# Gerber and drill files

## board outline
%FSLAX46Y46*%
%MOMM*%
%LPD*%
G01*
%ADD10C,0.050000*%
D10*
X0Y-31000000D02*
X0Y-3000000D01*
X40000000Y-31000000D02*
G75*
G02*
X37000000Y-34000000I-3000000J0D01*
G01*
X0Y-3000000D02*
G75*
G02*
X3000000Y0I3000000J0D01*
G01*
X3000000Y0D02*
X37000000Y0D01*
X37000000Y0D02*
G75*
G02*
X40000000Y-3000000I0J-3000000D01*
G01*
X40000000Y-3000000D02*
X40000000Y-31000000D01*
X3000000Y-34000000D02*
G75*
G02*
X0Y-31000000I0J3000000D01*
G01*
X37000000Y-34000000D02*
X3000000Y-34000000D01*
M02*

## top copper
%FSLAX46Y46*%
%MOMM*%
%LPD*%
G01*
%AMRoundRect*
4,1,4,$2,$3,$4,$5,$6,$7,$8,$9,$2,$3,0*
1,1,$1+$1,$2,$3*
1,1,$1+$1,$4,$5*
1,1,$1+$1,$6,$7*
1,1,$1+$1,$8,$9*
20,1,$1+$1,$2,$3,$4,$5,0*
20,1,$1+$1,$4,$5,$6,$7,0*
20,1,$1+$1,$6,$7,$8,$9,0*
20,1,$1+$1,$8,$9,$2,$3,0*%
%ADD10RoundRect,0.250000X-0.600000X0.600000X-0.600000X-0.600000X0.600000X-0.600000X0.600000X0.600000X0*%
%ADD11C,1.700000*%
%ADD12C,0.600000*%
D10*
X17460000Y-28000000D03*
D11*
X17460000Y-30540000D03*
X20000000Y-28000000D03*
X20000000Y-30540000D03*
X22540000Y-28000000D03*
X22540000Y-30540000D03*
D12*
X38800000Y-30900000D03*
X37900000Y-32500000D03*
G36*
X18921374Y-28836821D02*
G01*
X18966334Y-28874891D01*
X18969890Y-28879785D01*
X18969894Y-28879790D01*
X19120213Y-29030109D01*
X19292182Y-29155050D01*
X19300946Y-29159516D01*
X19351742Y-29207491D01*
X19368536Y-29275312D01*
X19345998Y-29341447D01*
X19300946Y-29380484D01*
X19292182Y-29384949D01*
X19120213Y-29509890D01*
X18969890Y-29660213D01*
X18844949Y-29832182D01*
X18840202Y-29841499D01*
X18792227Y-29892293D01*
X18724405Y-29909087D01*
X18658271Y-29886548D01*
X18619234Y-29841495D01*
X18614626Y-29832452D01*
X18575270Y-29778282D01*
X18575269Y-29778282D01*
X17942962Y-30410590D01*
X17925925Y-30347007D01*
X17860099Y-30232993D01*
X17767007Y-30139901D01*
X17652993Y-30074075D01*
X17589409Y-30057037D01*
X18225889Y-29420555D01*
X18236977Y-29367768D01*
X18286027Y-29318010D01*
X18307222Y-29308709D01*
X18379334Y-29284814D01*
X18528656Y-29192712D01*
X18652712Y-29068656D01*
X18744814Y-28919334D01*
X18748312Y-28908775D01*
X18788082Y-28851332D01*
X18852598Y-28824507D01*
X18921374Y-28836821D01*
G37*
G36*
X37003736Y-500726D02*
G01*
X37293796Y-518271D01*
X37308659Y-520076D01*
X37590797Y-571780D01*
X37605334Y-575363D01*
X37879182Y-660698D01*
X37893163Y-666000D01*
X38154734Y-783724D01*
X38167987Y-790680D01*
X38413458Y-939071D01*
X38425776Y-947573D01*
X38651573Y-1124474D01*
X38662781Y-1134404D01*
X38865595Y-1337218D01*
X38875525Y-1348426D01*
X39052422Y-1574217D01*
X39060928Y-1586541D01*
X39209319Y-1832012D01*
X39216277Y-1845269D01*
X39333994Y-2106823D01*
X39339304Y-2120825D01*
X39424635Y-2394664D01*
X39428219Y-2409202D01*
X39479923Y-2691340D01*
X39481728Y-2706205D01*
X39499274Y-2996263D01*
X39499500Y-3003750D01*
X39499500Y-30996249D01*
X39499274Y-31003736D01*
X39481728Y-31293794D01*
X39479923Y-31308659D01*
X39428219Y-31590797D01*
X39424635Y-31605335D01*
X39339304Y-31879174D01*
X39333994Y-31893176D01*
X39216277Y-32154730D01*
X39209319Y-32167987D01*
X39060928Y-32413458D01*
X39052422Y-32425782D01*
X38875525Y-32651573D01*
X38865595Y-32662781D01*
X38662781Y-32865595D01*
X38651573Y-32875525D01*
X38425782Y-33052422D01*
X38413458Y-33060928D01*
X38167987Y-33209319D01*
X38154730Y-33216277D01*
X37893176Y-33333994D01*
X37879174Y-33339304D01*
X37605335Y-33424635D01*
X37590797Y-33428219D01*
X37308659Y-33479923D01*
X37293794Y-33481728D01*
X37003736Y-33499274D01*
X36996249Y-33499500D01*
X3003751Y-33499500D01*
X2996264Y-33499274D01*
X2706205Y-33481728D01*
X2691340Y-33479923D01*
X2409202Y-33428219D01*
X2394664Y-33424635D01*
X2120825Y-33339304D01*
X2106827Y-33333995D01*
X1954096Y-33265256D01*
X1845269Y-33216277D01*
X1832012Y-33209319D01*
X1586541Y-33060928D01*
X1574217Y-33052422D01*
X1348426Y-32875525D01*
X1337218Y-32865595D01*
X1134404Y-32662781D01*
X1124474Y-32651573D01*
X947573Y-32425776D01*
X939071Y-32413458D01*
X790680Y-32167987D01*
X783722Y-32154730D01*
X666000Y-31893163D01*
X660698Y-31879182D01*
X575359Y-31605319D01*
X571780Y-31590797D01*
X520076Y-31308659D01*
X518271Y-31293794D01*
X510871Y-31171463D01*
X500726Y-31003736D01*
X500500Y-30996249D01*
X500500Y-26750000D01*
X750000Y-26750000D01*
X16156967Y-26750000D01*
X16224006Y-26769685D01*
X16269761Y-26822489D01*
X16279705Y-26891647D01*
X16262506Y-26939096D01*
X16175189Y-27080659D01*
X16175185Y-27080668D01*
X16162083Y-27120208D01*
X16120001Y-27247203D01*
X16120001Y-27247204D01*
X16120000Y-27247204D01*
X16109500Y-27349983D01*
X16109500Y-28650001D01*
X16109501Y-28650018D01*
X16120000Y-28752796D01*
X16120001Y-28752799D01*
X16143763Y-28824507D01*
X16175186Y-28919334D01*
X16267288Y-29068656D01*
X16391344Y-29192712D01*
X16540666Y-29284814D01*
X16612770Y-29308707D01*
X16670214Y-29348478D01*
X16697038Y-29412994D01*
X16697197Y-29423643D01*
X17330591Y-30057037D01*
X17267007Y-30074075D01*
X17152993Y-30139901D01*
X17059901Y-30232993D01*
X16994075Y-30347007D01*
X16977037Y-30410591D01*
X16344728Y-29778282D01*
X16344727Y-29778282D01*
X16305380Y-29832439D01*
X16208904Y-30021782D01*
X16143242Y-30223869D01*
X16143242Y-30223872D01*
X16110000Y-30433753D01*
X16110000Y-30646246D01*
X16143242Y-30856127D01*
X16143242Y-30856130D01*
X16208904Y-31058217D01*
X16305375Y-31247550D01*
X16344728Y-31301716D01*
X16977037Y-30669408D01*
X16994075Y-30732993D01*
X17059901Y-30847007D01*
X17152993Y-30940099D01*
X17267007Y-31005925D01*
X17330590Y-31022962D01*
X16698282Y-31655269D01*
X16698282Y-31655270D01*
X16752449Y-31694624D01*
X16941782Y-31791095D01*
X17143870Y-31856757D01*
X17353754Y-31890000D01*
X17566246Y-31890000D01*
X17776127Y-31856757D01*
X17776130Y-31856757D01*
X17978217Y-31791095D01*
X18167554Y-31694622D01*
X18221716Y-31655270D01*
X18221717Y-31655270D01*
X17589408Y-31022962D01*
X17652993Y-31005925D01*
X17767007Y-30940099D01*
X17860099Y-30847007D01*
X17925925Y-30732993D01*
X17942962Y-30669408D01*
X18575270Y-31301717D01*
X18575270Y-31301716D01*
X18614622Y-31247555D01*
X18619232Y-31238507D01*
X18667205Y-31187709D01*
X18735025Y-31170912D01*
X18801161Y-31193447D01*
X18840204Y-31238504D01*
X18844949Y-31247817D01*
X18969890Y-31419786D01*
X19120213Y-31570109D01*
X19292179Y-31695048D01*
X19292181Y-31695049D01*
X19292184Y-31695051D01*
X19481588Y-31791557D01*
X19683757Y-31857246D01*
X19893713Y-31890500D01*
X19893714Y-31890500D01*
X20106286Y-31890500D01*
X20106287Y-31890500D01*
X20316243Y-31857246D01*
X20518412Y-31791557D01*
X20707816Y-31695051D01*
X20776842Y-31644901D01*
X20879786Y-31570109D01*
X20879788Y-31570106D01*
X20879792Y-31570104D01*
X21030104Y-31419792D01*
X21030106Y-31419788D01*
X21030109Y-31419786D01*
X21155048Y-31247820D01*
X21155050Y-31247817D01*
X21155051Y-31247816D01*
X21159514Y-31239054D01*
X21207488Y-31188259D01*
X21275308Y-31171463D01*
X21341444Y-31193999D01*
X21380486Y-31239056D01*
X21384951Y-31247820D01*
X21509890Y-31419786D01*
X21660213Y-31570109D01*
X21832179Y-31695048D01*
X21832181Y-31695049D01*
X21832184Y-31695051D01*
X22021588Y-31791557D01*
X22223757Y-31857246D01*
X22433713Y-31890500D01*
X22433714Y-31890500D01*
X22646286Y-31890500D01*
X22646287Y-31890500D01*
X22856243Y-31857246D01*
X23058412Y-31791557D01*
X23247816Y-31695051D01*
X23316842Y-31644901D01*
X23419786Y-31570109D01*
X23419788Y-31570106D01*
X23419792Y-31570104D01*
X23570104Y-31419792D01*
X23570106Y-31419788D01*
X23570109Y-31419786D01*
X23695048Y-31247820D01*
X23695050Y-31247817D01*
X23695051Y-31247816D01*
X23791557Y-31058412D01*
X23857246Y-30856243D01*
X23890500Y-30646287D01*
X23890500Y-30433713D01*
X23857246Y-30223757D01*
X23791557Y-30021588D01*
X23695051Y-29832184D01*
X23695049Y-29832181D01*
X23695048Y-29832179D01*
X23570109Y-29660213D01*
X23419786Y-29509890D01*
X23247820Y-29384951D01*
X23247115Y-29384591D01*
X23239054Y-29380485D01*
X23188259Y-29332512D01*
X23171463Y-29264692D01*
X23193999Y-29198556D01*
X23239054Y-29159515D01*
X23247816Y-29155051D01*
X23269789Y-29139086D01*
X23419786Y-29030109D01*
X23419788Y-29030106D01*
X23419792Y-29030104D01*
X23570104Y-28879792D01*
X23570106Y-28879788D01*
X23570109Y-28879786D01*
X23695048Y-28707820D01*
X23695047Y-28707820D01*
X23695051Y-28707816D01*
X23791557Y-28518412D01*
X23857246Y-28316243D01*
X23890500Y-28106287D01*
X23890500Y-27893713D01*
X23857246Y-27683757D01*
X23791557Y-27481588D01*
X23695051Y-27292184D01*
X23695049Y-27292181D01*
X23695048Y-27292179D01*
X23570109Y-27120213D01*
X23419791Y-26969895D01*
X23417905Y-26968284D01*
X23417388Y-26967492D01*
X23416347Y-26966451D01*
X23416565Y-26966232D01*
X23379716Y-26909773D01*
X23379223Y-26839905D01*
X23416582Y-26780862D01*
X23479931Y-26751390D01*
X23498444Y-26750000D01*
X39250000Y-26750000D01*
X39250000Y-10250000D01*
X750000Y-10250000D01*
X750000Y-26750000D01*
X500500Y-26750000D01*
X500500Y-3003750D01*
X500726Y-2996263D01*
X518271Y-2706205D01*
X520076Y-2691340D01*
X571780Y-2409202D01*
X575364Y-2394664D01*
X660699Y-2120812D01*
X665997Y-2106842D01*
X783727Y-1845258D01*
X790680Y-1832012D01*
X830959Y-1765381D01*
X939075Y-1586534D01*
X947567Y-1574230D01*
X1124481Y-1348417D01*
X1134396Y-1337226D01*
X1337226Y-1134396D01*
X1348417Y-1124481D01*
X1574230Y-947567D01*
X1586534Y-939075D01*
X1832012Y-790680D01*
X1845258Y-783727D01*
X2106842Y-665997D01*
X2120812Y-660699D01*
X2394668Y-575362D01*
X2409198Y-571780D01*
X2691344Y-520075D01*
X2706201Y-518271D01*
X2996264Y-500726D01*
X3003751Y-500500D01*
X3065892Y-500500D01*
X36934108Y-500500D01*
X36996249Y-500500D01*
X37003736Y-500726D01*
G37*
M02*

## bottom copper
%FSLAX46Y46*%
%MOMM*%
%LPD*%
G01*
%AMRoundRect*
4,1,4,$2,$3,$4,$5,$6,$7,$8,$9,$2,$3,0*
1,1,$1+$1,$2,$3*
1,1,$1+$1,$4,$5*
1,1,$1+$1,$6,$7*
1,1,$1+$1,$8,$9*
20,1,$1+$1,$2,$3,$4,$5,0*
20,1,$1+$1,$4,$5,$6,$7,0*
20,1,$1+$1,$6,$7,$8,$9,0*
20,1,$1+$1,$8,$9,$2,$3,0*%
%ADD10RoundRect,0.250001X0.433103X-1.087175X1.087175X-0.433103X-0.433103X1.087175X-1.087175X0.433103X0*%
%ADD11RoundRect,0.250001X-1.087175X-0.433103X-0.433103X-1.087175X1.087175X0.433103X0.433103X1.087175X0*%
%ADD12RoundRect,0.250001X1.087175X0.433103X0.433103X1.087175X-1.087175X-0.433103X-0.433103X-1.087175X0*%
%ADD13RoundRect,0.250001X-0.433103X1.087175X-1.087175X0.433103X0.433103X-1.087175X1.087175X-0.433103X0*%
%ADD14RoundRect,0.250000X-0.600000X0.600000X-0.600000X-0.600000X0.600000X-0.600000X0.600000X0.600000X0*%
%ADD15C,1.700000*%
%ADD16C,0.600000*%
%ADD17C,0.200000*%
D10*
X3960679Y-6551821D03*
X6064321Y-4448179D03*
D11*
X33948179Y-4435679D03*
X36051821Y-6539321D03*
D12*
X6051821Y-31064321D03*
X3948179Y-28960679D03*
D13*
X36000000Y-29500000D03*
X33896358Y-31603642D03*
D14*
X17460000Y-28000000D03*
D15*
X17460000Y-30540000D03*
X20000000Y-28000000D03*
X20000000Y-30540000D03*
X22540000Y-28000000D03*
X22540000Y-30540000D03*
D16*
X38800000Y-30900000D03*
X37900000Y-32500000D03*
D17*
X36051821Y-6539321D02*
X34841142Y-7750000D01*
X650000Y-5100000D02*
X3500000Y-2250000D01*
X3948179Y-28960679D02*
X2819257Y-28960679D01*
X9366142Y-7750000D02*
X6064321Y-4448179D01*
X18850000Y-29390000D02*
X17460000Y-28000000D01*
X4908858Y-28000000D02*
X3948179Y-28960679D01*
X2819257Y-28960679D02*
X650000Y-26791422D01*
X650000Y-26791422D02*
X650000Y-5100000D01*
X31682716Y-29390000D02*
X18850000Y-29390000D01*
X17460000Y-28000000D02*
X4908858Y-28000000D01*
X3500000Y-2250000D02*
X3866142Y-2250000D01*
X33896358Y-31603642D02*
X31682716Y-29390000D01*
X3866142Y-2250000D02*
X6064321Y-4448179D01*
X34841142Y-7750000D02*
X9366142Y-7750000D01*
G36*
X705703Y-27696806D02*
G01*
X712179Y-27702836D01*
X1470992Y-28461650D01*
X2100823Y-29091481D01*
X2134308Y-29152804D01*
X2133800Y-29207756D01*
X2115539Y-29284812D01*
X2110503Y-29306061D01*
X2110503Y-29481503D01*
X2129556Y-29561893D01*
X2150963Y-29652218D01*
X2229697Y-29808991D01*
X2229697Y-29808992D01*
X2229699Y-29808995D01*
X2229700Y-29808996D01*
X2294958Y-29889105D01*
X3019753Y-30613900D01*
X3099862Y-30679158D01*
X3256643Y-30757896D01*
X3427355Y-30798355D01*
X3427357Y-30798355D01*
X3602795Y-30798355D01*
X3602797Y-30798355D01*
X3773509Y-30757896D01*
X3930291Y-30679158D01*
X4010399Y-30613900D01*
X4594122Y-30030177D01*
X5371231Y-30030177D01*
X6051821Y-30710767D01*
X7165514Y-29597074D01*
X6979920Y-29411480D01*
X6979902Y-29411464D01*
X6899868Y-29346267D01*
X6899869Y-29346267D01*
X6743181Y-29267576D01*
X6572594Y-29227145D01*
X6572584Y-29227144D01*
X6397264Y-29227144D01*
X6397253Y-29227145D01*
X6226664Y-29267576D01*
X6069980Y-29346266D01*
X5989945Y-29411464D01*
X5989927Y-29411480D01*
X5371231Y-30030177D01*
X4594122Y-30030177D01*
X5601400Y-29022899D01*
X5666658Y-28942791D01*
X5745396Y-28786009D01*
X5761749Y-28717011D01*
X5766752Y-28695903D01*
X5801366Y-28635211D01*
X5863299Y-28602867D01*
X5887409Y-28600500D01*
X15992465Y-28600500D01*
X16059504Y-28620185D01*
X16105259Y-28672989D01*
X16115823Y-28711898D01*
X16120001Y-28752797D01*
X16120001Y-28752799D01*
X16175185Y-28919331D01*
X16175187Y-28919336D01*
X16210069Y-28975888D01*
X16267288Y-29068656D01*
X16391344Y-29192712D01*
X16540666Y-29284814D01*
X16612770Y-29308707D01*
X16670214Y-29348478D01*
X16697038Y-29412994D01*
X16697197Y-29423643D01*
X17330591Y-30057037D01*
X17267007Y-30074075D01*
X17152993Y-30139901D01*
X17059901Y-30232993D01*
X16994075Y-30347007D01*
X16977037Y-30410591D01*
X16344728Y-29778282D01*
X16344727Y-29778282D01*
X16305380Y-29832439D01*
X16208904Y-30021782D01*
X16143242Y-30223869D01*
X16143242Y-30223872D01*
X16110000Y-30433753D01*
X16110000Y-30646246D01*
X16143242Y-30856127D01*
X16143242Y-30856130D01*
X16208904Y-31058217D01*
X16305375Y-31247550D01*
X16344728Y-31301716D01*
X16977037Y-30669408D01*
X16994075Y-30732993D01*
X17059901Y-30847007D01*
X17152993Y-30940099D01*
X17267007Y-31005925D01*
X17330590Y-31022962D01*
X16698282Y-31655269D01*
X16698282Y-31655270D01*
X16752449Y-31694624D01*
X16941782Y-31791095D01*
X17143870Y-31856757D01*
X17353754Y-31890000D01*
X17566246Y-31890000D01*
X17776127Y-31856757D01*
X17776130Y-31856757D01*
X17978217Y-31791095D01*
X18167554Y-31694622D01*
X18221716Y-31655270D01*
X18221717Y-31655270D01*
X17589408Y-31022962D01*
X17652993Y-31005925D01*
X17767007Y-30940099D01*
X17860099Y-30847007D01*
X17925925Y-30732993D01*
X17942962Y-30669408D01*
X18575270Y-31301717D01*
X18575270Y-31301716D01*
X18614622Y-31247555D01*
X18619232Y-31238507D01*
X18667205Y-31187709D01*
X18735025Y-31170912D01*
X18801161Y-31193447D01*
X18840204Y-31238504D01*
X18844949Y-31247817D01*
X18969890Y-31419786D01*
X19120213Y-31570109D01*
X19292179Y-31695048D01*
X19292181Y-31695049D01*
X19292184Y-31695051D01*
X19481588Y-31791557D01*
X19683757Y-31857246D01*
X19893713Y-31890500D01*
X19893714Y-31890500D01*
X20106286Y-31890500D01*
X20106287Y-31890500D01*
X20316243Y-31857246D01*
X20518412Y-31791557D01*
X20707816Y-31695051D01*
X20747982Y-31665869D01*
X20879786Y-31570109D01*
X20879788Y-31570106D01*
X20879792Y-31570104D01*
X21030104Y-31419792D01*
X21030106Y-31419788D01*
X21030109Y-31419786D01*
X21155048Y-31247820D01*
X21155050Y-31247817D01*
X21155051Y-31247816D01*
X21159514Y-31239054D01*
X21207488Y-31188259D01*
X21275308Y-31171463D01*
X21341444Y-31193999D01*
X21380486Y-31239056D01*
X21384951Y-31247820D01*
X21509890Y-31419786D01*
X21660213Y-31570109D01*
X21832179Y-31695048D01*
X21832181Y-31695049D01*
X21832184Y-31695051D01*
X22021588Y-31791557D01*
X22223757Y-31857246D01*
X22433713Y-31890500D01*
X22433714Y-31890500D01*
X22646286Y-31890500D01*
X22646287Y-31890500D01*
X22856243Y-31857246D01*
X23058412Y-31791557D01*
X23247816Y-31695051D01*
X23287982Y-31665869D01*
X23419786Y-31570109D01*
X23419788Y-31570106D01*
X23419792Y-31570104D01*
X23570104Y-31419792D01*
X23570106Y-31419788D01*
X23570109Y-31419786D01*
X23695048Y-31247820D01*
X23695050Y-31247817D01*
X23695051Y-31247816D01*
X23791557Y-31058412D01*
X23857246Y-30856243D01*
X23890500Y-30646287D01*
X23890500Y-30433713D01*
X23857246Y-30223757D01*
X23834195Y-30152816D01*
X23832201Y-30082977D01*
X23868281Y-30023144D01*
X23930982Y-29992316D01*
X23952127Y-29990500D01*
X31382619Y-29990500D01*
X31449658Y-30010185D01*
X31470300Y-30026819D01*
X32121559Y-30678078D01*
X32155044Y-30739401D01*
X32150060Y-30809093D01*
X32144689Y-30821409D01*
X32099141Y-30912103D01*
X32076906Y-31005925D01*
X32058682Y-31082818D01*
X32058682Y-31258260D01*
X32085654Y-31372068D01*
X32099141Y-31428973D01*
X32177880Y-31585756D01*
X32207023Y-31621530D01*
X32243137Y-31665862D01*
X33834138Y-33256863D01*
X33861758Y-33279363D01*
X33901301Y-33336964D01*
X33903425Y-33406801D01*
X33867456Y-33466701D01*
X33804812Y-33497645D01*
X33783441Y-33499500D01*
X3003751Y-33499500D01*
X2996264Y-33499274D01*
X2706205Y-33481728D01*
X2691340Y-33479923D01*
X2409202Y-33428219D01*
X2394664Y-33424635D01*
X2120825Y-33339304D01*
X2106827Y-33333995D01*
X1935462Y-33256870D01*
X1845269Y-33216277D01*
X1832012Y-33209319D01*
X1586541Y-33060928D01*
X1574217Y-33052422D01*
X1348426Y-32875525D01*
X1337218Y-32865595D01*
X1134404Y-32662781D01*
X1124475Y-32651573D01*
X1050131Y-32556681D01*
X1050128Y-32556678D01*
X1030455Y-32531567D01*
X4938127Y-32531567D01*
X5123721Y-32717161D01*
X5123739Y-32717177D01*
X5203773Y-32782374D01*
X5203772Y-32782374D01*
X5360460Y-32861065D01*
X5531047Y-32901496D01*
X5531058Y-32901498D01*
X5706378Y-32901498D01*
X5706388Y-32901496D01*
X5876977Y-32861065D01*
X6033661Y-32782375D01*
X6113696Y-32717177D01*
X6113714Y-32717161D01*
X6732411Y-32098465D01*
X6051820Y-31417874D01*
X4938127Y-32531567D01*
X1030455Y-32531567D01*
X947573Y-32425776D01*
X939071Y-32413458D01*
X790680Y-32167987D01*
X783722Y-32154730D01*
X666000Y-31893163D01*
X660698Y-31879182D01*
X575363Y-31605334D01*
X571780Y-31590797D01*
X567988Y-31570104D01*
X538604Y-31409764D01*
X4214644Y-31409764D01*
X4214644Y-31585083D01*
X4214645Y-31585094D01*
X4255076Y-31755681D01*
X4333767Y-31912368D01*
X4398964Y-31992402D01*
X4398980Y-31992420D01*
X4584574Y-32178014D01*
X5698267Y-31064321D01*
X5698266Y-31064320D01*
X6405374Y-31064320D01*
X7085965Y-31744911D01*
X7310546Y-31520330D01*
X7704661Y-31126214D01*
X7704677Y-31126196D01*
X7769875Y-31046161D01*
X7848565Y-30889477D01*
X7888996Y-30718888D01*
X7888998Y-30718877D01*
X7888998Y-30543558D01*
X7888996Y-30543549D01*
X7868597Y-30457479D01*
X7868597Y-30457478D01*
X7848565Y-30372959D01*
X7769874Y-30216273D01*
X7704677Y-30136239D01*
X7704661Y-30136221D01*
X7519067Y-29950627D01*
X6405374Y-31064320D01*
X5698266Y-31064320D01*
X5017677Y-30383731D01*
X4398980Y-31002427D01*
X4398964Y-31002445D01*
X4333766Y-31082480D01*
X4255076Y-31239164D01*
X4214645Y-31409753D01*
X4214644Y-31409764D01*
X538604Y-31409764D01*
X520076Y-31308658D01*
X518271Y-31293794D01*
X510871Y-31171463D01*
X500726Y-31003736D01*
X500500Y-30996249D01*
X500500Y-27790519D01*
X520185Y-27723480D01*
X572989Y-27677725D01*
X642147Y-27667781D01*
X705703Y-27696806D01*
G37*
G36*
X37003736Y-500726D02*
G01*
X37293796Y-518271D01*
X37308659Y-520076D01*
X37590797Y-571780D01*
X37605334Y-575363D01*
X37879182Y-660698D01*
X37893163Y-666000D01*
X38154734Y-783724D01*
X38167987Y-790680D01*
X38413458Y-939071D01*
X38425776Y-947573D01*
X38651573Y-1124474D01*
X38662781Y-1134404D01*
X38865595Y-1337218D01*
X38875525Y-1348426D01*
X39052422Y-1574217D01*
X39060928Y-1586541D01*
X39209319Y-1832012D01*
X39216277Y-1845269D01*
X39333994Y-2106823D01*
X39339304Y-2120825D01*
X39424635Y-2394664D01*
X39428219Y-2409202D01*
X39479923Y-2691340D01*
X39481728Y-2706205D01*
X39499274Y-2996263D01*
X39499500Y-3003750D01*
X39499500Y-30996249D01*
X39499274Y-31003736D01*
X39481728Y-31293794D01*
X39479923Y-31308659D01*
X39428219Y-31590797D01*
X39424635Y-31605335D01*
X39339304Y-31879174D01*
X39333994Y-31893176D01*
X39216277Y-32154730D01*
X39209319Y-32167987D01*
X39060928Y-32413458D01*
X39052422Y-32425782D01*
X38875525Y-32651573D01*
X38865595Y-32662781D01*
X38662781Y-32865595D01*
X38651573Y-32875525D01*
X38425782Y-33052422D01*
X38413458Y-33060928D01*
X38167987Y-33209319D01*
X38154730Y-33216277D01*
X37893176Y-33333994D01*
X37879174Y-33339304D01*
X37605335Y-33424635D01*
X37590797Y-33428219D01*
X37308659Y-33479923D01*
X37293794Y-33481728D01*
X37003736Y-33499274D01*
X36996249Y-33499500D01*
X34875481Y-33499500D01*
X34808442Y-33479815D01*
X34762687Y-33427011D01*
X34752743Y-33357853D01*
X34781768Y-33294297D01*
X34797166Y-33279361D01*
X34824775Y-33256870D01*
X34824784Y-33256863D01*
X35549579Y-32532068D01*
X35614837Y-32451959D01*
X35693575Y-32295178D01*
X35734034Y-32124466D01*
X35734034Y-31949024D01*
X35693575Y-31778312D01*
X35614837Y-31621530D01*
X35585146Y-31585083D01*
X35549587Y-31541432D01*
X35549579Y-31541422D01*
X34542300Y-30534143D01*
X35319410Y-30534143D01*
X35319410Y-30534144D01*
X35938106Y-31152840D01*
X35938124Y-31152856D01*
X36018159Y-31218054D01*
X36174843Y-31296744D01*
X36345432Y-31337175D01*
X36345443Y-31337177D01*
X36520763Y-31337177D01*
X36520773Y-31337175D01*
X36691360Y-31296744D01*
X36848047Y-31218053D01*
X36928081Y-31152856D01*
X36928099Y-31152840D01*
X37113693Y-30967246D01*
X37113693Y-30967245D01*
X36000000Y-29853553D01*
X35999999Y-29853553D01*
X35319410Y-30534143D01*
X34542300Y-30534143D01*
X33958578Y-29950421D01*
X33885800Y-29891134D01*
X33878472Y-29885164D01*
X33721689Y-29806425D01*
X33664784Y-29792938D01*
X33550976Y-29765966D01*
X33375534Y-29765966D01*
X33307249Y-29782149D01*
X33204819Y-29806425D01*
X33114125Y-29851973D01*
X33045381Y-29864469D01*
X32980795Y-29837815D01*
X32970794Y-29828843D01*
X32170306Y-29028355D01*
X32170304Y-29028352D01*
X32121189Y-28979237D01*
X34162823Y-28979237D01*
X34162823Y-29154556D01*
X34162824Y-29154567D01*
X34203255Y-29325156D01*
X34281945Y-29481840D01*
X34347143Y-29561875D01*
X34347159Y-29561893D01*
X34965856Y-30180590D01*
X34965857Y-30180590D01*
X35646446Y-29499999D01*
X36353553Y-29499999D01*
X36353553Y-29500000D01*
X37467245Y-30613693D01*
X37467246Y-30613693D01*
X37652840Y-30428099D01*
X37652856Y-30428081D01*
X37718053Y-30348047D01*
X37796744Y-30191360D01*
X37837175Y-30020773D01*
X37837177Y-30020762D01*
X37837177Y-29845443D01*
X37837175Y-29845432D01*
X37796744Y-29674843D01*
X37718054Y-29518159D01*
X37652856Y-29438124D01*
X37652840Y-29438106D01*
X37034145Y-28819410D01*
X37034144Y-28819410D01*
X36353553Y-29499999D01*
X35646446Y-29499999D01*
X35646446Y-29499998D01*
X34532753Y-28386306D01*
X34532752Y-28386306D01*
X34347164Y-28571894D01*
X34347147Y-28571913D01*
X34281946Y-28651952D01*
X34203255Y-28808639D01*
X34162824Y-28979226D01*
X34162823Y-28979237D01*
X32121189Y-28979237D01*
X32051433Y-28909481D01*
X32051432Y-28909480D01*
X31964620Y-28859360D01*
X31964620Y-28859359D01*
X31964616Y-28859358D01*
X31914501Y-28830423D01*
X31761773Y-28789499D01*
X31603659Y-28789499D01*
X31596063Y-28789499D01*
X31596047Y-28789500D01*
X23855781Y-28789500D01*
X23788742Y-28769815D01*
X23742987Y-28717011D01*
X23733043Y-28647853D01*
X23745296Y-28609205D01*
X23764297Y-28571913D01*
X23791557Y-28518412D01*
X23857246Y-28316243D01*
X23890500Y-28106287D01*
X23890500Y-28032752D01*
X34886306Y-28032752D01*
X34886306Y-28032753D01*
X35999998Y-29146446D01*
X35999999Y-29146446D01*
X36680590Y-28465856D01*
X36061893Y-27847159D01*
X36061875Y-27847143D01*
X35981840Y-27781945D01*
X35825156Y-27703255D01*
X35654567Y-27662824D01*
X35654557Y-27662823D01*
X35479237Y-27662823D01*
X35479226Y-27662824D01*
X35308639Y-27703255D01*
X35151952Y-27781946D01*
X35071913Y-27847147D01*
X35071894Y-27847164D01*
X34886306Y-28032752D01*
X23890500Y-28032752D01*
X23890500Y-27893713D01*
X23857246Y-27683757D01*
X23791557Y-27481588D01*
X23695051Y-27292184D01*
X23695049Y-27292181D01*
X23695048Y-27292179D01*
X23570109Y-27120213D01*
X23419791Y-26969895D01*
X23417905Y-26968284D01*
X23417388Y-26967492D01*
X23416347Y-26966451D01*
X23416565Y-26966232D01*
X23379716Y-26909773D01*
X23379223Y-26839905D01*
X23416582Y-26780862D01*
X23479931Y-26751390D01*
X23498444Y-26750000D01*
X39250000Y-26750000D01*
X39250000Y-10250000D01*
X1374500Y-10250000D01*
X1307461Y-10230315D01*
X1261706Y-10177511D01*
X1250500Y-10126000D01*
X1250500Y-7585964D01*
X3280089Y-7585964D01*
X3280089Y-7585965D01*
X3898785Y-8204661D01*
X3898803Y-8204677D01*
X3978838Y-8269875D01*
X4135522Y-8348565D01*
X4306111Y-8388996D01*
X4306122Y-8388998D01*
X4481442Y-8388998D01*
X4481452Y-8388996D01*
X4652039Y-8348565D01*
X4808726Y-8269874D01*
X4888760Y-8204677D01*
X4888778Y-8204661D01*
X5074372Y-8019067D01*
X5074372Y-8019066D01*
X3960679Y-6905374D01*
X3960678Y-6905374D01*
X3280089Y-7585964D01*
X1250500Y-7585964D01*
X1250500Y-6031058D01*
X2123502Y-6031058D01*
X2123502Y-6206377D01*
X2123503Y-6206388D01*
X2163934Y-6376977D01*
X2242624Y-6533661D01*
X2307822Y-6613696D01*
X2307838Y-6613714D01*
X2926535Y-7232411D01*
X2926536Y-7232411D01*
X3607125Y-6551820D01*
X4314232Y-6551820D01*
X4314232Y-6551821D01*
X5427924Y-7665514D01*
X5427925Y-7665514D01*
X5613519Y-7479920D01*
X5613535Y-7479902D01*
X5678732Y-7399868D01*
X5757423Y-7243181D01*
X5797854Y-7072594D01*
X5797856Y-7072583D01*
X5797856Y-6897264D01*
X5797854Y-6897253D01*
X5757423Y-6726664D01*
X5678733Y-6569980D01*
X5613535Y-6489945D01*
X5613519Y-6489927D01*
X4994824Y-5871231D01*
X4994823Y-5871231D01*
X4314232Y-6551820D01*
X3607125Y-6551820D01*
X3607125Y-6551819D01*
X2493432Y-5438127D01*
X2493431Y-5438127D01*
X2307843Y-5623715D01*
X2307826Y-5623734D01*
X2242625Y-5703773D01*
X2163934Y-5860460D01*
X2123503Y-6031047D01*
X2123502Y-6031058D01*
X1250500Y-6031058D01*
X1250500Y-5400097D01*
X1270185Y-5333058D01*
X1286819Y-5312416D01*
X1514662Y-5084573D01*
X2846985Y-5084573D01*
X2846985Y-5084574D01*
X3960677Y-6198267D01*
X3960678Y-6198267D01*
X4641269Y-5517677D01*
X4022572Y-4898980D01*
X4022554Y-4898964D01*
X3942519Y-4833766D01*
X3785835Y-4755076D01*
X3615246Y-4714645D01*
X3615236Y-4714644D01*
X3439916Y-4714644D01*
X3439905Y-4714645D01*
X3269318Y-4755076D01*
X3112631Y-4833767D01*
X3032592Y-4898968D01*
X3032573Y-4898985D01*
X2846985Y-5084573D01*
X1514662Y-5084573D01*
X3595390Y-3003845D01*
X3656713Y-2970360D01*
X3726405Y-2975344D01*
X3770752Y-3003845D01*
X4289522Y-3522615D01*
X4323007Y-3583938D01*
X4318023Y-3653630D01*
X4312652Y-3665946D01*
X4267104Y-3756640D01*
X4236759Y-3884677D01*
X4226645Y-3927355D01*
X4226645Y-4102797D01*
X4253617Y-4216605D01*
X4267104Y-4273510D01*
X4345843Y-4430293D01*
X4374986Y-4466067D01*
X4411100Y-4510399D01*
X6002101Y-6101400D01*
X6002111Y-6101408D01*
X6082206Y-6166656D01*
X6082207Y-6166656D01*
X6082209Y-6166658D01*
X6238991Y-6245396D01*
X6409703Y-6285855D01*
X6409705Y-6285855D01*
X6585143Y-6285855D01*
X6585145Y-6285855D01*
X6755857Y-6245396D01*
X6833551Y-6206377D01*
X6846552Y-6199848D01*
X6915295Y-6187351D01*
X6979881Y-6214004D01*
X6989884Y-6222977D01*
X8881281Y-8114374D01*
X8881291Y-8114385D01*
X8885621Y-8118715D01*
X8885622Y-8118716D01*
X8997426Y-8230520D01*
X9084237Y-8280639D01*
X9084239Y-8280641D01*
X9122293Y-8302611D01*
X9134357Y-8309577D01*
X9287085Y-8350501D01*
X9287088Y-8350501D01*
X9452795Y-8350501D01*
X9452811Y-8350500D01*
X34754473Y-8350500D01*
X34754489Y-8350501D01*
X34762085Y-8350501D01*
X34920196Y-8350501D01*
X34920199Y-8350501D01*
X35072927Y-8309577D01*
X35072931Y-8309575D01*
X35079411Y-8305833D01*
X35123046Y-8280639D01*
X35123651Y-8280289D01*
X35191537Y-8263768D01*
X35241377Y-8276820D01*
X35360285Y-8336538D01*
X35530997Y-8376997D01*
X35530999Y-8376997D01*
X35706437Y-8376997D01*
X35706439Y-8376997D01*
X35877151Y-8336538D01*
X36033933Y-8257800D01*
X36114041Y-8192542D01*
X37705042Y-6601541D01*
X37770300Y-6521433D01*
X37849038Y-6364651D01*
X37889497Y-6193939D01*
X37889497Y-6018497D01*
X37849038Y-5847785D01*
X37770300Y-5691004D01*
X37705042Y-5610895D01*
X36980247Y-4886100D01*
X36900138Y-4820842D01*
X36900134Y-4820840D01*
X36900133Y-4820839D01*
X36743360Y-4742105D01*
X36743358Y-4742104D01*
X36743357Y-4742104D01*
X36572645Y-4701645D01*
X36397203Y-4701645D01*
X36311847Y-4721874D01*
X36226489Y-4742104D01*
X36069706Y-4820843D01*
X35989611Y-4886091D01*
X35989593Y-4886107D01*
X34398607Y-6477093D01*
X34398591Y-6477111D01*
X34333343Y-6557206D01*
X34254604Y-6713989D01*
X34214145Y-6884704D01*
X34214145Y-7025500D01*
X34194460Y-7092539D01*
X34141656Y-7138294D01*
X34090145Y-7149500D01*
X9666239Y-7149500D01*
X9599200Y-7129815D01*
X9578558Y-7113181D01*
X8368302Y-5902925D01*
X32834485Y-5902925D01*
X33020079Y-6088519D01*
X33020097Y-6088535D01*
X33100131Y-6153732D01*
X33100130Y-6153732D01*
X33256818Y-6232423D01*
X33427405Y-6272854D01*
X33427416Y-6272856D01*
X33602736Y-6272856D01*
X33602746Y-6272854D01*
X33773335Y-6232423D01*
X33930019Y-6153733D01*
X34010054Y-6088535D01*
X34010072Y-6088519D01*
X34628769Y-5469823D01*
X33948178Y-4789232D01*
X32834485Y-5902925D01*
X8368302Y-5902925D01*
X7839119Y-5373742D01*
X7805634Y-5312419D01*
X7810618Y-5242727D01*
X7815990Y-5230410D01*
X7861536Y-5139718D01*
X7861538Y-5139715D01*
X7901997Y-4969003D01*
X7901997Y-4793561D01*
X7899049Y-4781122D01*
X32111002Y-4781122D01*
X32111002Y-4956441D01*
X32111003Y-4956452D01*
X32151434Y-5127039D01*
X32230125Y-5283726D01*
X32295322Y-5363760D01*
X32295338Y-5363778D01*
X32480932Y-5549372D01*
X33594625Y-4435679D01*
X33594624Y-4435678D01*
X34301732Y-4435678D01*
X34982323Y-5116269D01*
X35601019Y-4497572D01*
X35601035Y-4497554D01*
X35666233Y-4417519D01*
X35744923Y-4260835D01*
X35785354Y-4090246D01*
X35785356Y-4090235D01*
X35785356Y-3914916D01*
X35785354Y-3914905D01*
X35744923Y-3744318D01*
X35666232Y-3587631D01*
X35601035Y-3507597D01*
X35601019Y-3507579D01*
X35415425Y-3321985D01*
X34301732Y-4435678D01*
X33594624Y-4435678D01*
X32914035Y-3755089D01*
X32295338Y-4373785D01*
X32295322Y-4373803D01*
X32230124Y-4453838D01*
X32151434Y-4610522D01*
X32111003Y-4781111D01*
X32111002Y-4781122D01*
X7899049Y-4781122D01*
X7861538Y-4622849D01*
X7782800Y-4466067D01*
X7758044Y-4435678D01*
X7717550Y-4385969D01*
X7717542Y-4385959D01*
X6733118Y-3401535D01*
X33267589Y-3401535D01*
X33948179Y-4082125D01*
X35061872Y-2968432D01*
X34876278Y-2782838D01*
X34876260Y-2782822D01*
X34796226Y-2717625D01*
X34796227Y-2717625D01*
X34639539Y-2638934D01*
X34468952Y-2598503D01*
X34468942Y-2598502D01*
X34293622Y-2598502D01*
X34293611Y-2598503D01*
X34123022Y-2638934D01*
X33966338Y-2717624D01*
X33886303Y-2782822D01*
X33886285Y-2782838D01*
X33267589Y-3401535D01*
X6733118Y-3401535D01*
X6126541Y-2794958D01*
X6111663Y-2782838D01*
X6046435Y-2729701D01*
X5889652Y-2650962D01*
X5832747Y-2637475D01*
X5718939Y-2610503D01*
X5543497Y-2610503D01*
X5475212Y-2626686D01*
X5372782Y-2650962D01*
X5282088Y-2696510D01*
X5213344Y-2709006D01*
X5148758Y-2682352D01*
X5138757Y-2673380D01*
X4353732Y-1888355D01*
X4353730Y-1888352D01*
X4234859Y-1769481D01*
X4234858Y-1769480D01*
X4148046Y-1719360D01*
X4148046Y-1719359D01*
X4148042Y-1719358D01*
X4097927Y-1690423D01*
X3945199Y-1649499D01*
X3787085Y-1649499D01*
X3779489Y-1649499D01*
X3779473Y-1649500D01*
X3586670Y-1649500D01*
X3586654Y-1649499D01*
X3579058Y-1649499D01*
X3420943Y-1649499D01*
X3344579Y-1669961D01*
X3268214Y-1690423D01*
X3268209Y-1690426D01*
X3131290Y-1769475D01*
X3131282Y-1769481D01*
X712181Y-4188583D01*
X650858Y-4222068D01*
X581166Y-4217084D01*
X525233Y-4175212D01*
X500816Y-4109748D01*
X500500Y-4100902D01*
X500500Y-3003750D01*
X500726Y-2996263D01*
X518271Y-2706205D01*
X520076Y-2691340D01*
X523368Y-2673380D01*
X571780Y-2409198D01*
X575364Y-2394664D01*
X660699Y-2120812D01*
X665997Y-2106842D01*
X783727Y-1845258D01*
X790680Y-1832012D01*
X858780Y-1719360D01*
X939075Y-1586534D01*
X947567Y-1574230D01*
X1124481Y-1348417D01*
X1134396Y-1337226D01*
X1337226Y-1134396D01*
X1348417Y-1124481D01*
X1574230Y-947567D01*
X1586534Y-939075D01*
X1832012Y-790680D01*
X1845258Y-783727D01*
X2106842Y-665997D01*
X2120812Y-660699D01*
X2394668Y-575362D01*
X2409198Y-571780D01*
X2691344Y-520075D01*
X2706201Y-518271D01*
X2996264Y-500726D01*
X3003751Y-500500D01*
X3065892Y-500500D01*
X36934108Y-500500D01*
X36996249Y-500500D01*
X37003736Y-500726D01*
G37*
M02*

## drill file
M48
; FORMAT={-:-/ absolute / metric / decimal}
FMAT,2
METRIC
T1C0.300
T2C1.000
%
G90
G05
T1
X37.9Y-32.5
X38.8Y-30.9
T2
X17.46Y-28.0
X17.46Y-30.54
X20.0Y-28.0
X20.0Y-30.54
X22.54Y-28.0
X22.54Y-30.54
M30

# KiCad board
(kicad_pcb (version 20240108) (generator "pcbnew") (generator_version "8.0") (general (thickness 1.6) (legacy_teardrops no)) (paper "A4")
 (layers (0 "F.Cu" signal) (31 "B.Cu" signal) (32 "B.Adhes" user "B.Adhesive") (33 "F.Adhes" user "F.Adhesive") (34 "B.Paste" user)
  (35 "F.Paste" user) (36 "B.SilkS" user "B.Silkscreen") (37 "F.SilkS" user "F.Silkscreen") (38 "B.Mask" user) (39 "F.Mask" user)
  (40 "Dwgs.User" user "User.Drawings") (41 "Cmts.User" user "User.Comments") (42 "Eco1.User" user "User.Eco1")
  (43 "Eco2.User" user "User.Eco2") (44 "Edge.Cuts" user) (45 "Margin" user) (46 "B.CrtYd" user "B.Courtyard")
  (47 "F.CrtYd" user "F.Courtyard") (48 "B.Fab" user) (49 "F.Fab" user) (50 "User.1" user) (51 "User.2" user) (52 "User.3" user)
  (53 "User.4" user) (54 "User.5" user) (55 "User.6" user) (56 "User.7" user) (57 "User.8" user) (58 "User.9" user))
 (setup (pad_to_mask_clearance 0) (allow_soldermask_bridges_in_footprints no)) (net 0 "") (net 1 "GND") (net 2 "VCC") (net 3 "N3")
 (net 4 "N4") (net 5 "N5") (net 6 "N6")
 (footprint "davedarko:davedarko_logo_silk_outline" (layer "F.Cu") (at 36.5 30)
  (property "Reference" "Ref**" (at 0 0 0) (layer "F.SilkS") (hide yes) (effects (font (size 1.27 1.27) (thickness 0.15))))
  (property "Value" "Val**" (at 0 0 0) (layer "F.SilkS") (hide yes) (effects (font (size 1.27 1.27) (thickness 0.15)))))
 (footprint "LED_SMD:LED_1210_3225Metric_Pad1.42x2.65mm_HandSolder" (layer "B.Cu") (at 5.0125 5.5 45)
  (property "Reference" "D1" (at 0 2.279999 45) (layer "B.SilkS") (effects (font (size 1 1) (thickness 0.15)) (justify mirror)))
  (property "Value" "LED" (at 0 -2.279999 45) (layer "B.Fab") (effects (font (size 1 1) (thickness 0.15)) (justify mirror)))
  (pad "1" smd roundrect (at -1.4875 0 45) (size 1.425 2.65) (layers "B.Cu" "B.Paste" "B.Mask") (roundrect_rratio 0.175439) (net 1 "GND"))
  (pad "2" smd roundrect (at 1.4875 0 45) (size 1.425 2.65) (layers "B.Cu" "B.Paste" "B.Mask") (roundrect_rratio 0.175439) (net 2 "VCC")))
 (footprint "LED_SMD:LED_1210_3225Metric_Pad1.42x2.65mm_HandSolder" (layer "B.Cu") (at 35 5.4875 -45)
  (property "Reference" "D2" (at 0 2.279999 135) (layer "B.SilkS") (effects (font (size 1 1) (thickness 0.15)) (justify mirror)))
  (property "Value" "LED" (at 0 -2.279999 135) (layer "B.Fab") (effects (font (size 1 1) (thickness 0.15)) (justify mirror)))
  (pad "1" smd roundrect (at -1.4875 0 315) (size 1.425 2.65) (layers "B.Cu" "B.Paste" "B.Mask") (roundrect_rratio 0.175439) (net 1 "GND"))
  (pad "2" smd roundrect (at 1.4875 0 315) (size 1.425 2.65) (layers "B.Cu" "B.Paste" "B.Mask") (roundrect_rratio 0.175439) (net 2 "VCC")))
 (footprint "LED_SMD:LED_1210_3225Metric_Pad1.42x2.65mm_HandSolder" (layer "B.Cu") (at 5 30.0125 135)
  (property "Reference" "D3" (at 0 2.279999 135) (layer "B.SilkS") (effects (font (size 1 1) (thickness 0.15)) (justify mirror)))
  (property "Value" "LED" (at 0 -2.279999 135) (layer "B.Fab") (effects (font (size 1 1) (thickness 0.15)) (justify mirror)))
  (pad "1" smd roundrect (at -1.4875 0 135) (size 1.425 2.65) (layers "B.Cu" "B.Paste" "B.Mask") (roundrect_rratio 0.175439) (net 1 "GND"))
  (pad "2" smd roundrect (at 1.4875 0 135) (size 1.425 2.65) (layers "B.Cu" "B.Paste" "B.Mask") (roundrect_rratio 0.175439) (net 2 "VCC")))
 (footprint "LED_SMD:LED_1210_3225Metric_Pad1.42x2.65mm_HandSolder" (layer "B.Cu") (at 34.948179 30.551821 -135)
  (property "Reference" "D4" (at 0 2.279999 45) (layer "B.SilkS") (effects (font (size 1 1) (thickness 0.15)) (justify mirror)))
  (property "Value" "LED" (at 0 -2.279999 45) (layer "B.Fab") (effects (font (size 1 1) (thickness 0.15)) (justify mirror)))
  (pad "1" smd roundrect (at -1.4875 0 225) (size 1.425 2.65) (layers "B.Cu" "B.Paste" "B.Mask") (roundrect_rratio 0.175439) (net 1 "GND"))
  (pad "2" smd roundrect (at 1.4875 0 225) (size 1.425 2.65) (layers "B.Cu" "B.Paste" "B.Mask") (roundrect_rratio 0.175439) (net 2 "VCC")))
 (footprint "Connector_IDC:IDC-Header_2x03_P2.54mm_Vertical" (layer "B.Cu") (at 17.46 28 -90)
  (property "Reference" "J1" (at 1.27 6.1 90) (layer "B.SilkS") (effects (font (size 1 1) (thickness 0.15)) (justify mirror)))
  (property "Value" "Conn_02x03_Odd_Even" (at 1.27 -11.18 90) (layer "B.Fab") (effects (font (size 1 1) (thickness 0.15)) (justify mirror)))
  (pad "1" thru_hole roundrect (at 0 0 270) (size 1.7 1.7) (drill 1) (layers "*.Cu" "*.Mask") (remove_unused_layers no)
   (roundrect_rratio 0.147059) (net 2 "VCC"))
  (pad "2" thru_hole circle (at 2.54 0 270) (size 1.7 1.7) (drill 1) (layers "*.Cu" "*.Mask") (remove_unused_layers no) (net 1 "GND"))
  (pad "3" thru_hole circle (at 0 -2.54 270) (size 1.7 1.7) (drill 1) (layers "*.Cu" "*.Mask") (remove_unused_layers no) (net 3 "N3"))
  (pad "4" thru_hole circle (at 2.54 -2.54 270) (size 1.7 1.7) (drill 1) (layers "*.Cu" "*.Mask") (remove_unused_layers no) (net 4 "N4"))
  (pad "5" thru_hole circle (at 0 -5.08 270) (size 1.7 1.7) (drill 1) (layers "*.Cu" "*.Mask") (remove_unused_layers no) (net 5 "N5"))
  (pad "6" thru_hole circle (at 2.54 -5.08 270) (size 1.7 1.7) (drill 1) (layers "*.Cu" "*.Mask") (remove_unused_layers no) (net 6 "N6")))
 (gr_line (start 0 31) (end 0 3) (stroke (width 0.05) (type default)) (layer "Edge.Cuts"))
 (gr_arc (start 40 31) (mid 39.12132 33.12132) (end 37 34) (stroke (width 0.05) (type default)) (layer "Edge.Cuts"))
 (gr_arc (start 0 3) (mid 0.87868 0.87868) (end 3 0) (stroke (width 0.05) (type default)) (layer "Edge.Cuts"))
 (gr_line (start 3 0) (end 37 0) (stroke (width 0.05) (type default)) (layer "Edge.Cuts"))
 (gr_arc (start 37 0) (mid 39.12132 0.87868) (end 40 3) (stroke (width 0.05) (type default)) (layer "Edge.Cuts"))
 (gr_line (start 40 3) (end 40 31) (stroke (width 0.05) (type default)) (layer "Edge.Cuts"))
 (gr_arc (start 3 34) (mid 0.87868 33.12132) (end 0 31) (stroke (width 0.05) (type default)) (layer "Edge.Cuts"))
 (gr_line (start 37 34) (end 3 34) (stroke (width 0.05) (type default)) (layer "Edge.Cuts"))
 (segment (start 36.051821 6.539321) (end 34.841142 7.75) (width 0.2) (layer "B.Cu") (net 2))
 (segment (start 0.65 5.1) (end 3.5 2.25) (width 0.2) (layer "B.Cu") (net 2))
 (segment (start 3.948179 28.960679) (end 2.819257 28.960679) (width 0.2) (layer "B.Cu") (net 2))
 (segment (start 9.366142 7.75) (end 6.064321 4.448179) (width 0.2) (layer "B.Cu") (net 2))
 (segment (start 18.85 29.39) (end 17.46 28) (width 0.2) (layer "B.Cu") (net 2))
 (segment (start 4.908858 28) (end 3.948179 28.960679) (width 0.2) (layer "B.Cu") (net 2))
 (segment (start 2.819257 28.960679) (end 0.65 26.791422) (width 0.2) (layer "B.Cu") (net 2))
 (segment (start 0.65 26.791422) (end 0.65 5.1) (width 0.2) (layer "B.Cu") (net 2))
 (segment (start 31.682716 29.39) (end 18.85 29.39) (width 0.2) (layer "B.Cu") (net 2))
 (segment (start 17.46 28) (end 4.908858 28) (width 0.2) (layer "B.Cu") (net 2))
 (segment (start 3.5 2.25) (end 3.866142 2.25) (width 0.2) (layer "B.Cu") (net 2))
 (segment (start 33.896358 31.603642) (end 31.682716 29.39) (width 0.2) (layer "B.Cu") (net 2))
 (segment (start 3.866142 2.25) (end 6.064321 4.448179) (width 0.2) (layer "B.Cu") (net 2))
 (segment (start 34.841142 7.75) (end 9.366142 7.75) (width 0.2) (layer "B.Cu") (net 2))
 (via (at 38.8 30.9) (size 0.6) (drill 0.3) (layers "F.Cu" "B.Cu") (free yes) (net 1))
 (via (at 37.9 32.5) (size 0.6) (drill 0.3) (layers "F.Cu" "B.Cu") (free yes) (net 1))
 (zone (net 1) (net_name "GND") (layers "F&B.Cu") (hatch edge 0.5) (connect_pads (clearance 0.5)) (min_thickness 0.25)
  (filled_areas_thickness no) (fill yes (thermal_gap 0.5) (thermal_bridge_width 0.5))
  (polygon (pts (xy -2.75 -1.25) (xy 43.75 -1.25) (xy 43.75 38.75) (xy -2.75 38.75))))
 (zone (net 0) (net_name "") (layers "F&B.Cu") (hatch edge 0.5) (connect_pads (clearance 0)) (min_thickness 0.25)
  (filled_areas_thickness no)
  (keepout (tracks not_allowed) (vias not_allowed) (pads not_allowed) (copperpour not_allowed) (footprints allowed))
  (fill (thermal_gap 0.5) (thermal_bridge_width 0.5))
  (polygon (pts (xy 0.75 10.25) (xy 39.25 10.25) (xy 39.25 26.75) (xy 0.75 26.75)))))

